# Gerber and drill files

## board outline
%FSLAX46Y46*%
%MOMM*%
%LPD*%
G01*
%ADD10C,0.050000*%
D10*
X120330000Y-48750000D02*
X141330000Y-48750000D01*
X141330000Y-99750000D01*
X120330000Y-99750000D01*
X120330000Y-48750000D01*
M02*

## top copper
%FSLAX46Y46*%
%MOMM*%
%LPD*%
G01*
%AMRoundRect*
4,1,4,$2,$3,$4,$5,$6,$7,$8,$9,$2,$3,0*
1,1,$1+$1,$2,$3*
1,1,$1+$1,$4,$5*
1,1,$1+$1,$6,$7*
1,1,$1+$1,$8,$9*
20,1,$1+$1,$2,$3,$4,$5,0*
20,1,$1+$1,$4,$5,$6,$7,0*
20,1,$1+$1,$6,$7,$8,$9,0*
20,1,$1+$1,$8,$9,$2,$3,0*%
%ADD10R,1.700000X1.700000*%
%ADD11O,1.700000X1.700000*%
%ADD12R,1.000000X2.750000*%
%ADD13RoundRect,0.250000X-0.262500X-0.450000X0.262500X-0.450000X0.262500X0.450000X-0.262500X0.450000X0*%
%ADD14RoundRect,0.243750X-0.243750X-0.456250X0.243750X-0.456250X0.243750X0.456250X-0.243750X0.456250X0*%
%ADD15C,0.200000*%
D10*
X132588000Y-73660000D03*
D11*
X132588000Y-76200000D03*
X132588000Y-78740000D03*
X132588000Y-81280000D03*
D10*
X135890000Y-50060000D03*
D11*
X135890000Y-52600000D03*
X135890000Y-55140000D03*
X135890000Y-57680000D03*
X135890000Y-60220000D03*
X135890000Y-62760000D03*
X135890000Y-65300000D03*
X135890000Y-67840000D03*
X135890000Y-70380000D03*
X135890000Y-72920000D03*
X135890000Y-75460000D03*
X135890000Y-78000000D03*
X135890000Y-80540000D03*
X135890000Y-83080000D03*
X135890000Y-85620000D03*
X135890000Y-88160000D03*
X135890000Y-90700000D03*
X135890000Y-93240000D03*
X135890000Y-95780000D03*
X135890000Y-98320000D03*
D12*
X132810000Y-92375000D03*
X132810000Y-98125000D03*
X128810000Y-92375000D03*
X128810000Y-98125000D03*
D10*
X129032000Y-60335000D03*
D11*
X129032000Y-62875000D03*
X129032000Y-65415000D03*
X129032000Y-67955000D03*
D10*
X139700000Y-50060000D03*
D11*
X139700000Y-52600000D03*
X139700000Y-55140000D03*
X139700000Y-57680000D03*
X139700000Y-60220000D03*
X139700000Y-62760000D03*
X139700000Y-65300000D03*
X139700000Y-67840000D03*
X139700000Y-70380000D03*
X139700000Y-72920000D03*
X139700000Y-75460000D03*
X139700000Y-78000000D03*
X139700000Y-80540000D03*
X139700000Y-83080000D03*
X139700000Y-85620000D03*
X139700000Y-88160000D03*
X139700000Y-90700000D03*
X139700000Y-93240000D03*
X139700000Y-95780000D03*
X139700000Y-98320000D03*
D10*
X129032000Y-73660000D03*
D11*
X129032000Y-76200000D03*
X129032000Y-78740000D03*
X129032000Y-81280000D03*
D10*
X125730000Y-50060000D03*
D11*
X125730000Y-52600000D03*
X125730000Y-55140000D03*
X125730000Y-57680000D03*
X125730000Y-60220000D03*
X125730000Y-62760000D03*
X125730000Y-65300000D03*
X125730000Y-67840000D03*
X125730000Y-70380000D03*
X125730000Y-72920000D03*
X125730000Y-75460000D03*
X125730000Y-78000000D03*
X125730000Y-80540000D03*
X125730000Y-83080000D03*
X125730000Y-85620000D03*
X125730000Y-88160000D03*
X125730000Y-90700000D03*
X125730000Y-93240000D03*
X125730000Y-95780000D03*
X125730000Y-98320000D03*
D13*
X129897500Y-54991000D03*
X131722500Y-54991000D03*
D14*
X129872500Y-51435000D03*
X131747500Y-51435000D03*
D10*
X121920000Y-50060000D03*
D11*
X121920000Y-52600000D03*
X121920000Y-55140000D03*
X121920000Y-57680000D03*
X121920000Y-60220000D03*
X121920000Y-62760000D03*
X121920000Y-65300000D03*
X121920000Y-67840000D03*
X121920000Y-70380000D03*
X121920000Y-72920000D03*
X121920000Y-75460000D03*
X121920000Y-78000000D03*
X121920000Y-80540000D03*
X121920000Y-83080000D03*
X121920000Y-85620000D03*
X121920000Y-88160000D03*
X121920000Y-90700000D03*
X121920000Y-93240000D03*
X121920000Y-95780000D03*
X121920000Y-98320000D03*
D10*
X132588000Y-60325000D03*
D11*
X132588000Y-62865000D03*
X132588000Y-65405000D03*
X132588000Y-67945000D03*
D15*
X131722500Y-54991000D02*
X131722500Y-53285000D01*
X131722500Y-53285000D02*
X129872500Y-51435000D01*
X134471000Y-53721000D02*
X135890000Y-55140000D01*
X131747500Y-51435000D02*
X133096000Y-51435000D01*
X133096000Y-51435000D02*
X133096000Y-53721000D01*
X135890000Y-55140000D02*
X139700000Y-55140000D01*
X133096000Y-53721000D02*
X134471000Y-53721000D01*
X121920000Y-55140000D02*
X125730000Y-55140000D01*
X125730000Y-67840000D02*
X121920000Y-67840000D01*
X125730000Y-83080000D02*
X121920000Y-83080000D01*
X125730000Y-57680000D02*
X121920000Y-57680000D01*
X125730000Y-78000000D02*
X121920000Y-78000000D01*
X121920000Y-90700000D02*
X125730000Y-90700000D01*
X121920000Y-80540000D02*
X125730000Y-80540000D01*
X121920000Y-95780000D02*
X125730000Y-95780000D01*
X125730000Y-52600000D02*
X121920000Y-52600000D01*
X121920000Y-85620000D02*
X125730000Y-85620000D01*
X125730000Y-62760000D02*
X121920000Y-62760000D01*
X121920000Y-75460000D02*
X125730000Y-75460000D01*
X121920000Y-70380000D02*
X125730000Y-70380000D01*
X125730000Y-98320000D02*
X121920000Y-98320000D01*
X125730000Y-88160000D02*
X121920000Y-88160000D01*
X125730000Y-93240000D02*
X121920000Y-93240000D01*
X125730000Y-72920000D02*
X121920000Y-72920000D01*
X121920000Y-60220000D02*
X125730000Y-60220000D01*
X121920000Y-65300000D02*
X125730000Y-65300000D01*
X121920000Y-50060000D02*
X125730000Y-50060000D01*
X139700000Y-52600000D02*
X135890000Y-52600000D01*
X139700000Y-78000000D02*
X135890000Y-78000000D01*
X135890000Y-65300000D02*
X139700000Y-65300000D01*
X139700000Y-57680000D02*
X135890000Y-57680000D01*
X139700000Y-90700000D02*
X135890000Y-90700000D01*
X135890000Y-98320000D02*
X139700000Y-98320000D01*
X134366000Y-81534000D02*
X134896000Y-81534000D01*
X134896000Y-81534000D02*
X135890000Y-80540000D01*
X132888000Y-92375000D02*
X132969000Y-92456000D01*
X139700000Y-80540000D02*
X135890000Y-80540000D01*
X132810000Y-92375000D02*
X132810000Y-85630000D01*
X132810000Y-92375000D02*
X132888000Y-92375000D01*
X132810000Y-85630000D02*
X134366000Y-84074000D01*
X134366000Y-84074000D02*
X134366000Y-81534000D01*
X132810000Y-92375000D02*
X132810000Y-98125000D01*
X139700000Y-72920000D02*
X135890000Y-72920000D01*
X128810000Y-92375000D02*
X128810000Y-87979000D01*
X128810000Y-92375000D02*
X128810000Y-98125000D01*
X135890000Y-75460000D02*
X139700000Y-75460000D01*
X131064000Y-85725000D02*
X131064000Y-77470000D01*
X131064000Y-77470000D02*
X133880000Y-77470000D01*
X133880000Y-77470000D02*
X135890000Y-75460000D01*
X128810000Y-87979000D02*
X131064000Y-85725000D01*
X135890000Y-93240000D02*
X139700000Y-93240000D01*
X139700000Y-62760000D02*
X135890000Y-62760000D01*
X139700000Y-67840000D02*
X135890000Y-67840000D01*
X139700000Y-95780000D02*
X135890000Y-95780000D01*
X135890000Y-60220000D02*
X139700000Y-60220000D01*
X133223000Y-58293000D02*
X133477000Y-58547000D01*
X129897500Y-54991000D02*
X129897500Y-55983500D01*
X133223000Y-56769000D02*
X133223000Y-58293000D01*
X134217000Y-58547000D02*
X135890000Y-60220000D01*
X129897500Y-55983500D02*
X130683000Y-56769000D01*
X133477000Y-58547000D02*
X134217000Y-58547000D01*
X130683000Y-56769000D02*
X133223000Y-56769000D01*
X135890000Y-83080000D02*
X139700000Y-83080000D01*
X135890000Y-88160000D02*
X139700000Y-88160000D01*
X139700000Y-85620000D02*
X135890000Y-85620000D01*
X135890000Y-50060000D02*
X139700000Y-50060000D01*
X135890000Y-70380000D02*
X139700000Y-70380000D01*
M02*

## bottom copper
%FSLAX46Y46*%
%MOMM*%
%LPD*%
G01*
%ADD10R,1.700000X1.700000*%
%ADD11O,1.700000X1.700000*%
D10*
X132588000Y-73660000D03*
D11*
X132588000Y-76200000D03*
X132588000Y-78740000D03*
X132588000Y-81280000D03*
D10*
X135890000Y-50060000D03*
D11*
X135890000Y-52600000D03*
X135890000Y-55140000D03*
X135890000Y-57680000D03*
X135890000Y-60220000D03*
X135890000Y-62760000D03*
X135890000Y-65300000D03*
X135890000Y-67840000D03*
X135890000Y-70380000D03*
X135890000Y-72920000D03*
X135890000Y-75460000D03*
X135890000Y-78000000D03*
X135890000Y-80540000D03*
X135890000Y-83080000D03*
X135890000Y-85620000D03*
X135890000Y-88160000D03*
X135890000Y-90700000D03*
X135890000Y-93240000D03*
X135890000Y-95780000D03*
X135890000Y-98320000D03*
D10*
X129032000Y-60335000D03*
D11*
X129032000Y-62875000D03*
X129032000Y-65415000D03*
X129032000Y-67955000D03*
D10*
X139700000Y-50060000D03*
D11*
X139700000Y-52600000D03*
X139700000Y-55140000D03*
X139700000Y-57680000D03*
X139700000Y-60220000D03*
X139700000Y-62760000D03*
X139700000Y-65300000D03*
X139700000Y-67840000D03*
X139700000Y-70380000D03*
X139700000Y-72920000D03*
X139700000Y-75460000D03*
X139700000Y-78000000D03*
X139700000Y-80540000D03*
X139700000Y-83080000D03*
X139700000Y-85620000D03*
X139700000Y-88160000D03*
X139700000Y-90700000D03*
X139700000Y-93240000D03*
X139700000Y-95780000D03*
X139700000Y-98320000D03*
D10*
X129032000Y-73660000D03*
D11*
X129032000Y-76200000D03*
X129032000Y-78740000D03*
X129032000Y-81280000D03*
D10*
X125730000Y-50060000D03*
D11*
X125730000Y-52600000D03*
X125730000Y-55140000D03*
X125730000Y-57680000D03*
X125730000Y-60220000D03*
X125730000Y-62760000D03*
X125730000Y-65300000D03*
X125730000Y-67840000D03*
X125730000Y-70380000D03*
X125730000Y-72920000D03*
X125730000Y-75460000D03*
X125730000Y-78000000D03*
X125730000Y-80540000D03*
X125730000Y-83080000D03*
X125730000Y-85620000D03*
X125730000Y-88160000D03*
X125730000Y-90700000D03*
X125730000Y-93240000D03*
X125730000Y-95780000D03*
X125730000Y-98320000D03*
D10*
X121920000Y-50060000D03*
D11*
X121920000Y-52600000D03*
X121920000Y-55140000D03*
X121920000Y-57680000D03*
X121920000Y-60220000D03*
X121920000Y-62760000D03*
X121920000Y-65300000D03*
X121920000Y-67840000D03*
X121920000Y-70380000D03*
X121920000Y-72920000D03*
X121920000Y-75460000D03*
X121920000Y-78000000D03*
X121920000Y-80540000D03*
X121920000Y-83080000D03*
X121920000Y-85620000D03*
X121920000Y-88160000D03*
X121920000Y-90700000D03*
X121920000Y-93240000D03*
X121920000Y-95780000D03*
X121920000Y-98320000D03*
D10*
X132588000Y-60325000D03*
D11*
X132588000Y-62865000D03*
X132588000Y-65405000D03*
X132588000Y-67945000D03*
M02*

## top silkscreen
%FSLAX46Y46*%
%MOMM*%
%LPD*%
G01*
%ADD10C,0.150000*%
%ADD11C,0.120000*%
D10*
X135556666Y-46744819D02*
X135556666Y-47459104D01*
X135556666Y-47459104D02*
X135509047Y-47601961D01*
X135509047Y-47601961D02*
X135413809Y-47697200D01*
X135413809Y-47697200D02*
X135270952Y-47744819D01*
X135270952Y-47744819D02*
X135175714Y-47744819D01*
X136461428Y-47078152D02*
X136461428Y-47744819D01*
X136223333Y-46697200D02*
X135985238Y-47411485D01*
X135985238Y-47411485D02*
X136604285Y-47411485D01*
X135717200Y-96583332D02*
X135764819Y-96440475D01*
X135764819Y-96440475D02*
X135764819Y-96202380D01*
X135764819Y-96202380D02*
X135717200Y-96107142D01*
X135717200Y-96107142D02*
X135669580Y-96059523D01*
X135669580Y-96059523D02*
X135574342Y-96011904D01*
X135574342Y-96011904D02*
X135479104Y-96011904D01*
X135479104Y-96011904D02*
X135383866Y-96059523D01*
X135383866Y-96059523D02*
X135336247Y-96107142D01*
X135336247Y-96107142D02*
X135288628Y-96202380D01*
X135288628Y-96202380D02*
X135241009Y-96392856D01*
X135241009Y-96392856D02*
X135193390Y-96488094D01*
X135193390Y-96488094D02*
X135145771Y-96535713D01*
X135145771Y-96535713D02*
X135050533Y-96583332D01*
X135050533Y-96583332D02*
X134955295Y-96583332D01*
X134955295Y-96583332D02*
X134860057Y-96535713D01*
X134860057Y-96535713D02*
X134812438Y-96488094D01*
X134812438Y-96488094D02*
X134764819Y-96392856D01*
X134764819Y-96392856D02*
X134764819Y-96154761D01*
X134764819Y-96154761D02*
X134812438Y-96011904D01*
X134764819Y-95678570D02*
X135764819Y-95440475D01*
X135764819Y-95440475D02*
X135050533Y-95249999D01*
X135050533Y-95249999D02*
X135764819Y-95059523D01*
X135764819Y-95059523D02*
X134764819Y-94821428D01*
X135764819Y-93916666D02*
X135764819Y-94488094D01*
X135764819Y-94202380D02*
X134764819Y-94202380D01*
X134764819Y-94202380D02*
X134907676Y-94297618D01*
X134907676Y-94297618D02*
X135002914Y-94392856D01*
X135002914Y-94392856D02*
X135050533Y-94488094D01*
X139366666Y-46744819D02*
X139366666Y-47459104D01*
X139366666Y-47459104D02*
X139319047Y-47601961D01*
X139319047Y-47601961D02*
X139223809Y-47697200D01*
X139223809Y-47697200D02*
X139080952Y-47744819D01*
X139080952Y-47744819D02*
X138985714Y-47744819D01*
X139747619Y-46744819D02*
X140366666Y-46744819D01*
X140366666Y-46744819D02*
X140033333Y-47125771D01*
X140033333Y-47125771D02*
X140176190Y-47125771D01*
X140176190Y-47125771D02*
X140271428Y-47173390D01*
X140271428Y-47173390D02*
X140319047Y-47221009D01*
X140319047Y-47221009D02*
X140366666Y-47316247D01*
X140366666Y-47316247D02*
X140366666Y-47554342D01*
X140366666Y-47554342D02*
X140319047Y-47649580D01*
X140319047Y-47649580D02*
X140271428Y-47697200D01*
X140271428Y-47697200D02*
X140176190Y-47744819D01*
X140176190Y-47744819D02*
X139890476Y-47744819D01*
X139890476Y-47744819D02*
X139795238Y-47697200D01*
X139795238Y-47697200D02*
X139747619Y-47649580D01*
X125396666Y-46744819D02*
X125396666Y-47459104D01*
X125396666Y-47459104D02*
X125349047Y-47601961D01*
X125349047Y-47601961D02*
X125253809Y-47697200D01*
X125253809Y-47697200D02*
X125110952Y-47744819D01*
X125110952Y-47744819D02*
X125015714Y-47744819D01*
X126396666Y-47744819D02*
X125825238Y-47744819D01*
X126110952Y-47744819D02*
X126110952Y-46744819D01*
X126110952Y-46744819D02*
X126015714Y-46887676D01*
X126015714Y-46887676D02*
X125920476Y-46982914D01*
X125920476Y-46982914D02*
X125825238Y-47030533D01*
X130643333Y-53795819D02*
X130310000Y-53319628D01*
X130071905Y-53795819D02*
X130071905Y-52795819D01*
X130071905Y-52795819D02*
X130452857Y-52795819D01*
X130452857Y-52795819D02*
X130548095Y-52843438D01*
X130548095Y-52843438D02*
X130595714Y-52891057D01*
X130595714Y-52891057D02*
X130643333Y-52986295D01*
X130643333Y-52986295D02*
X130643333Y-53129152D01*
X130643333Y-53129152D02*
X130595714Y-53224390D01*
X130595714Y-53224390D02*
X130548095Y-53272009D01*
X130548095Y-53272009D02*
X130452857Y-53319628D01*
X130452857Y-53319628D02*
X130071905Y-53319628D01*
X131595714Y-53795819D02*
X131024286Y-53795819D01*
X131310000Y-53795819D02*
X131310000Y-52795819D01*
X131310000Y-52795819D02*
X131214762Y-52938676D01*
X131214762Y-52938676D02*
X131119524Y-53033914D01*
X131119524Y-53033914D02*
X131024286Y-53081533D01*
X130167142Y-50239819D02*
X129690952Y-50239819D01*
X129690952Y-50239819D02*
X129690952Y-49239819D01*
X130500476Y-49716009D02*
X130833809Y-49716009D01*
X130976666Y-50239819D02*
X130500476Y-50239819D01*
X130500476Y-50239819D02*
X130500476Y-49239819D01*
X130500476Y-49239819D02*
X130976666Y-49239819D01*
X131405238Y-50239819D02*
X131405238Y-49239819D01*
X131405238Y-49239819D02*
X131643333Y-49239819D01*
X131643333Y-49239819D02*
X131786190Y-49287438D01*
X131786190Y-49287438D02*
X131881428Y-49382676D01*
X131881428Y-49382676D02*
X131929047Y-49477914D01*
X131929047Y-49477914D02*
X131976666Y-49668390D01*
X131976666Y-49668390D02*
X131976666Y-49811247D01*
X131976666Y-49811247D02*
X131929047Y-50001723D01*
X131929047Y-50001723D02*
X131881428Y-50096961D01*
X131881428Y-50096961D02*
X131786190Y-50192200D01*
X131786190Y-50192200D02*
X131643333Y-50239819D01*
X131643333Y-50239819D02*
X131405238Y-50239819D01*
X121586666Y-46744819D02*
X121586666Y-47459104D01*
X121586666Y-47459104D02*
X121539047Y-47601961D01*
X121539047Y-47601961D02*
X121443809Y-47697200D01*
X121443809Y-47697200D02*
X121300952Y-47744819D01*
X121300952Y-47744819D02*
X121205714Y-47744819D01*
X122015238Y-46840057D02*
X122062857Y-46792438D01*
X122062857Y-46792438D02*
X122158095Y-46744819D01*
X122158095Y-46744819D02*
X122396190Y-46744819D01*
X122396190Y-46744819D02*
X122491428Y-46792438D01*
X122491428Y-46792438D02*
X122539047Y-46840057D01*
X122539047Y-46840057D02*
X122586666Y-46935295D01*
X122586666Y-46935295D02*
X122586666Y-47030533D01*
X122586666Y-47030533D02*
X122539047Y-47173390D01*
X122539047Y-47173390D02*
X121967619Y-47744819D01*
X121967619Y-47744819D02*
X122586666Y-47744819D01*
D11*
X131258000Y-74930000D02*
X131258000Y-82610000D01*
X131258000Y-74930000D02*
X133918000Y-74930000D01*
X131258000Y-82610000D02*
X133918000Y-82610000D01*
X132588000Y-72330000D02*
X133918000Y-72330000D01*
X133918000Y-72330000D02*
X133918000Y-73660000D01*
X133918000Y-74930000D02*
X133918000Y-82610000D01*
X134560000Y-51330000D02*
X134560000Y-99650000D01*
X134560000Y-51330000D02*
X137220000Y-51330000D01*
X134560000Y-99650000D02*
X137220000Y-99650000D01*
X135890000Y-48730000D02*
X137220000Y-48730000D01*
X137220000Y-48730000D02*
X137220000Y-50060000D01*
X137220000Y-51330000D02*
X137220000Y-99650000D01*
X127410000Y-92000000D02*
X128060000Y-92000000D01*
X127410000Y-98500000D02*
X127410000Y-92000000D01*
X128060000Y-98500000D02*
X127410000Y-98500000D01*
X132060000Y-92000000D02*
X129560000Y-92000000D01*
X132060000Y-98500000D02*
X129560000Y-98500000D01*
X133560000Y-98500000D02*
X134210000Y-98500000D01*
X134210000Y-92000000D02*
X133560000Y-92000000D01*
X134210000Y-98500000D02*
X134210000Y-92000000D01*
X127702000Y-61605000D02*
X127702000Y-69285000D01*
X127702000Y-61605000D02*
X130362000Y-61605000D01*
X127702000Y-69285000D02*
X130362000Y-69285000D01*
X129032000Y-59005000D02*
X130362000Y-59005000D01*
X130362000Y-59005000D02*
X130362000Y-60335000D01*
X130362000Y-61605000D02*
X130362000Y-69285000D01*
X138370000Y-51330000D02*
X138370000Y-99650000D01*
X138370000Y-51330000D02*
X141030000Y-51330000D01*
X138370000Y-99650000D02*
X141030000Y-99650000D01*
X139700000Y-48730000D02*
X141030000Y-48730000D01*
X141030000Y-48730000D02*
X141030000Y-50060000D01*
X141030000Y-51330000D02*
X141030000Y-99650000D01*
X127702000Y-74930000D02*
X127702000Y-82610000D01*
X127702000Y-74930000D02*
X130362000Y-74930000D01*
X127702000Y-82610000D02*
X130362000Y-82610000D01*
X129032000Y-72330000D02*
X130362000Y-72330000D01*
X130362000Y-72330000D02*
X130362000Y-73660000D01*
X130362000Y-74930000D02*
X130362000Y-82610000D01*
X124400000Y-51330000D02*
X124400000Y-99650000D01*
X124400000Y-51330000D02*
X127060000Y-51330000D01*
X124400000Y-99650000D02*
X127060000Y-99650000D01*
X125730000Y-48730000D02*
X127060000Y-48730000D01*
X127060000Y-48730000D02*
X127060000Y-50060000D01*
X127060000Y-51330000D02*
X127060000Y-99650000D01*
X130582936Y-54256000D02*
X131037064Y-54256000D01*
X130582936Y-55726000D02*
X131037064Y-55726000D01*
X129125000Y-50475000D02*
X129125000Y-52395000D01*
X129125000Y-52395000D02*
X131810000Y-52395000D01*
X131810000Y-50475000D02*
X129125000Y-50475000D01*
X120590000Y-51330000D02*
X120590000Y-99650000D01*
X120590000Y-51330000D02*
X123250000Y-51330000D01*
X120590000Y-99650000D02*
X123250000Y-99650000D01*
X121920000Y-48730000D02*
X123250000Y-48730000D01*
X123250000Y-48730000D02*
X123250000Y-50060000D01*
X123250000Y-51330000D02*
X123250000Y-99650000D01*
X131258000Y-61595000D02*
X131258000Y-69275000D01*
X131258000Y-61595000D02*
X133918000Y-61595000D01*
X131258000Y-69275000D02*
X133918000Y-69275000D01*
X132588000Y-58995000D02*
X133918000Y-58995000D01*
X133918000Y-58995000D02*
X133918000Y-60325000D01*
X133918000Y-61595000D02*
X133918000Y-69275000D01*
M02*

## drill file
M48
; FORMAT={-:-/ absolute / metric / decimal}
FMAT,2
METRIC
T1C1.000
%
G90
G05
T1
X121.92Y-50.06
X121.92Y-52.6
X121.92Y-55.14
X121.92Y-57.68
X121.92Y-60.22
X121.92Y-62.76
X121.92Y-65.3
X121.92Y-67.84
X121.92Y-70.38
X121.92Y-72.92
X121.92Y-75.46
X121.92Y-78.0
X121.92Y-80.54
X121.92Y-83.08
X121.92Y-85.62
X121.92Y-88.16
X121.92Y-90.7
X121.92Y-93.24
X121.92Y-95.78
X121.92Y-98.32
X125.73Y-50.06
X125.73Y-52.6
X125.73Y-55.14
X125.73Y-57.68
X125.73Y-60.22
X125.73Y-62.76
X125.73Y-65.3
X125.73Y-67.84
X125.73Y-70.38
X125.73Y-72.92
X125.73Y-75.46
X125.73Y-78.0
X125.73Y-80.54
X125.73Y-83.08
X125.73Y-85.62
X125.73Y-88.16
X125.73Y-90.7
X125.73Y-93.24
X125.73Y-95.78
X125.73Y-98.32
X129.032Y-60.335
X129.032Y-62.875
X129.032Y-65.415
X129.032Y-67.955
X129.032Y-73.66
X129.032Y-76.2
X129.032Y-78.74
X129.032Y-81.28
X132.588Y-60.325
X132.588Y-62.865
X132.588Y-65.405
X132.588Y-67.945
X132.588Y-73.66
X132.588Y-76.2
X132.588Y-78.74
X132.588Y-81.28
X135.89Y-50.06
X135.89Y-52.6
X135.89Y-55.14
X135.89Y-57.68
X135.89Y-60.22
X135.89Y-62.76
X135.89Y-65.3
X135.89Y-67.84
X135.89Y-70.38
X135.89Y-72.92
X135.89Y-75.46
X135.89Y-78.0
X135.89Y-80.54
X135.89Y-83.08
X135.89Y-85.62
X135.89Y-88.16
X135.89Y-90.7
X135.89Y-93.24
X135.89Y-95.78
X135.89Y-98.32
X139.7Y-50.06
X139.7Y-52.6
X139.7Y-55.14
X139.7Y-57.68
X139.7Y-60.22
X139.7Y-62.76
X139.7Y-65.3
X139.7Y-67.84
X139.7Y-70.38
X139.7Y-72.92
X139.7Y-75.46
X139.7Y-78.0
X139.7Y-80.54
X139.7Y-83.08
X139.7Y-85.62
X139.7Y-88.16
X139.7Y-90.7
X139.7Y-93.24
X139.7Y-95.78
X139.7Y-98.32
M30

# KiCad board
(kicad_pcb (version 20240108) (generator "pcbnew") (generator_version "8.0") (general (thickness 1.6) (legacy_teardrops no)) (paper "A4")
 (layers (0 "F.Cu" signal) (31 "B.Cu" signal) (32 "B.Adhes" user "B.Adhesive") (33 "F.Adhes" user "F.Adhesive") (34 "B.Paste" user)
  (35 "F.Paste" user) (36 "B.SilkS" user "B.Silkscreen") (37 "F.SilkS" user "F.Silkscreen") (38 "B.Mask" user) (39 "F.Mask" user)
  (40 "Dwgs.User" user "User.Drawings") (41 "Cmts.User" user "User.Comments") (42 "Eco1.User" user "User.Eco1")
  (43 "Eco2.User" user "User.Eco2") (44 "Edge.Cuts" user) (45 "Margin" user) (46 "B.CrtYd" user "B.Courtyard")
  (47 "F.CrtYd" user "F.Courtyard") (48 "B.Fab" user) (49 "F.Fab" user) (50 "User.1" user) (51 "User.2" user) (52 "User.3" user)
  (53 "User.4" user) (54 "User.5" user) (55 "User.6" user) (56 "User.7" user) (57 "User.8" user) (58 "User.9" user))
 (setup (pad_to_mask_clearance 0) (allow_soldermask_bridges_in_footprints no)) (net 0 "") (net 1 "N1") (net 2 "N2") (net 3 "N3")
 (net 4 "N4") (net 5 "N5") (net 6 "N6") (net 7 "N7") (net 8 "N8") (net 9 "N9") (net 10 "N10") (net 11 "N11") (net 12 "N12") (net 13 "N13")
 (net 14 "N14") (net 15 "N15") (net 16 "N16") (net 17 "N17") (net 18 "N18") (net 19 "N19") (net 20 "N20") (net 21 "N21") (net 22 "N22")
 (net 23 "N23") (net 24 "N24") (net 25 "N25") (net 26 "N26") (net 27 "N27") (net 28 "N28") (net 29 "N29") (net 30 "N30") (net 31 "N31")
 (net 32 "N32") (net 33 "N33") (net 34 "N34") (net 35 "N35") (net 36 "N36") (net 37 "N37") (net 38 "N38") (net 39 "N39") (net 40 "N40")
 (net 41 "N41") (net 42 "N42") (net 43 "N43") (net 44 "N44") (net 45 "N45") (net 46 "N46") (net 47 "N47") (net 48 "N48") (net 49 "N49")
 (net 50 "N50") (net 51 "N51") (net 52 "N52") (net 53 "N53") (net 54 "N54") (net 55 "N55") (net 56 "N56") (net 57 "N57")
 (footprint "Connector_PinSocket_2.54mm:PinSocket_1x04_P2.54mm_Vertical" (layer "F.Cu") (at 132.588 73.66)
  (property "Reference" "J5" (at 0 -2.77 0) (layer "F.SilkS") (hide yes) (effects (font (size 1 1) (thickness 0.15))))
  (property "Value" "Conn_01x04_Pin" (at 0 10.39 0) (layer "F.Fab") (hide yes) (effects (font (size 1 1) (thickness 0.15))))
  (fp_line (start -1.33 1.27) (end -1.33 8.95) (stroke (width 0.12) (type solid)) (layer "F.SilkS"))
  (fp_line (start -1.33 1.27) (end 1.33 1.27) (stroke (width 0.12) (type solid)) (layer "F.SilkS"))
  (fp_line (start -1.33 8.95) (end 1.33 8.95) (stroke (width 0.12) (type solid)) (layer "F.SilkS"))
  (fp_line (start 0 -1.33) (end 1.33 -1.33) (stroke (width 0.12) (type solid)) (layer "F.SilkS"))
  (fp_line (start 1.33 -1.33) (end 1.33 0) (stroke (width 0.12) (type solid)) (layer "F.SilkS"))
  (fp_line (start 1.33 1.27) (end 1.33 8.95) (stroke (width 0.12) (type solid)) (layer "F.SilkS"))
  (pad "1" thru_hole rect (at 0 0) (size 1.7 1.7) (drill 1) (layers "*.Cu" "*.Mask") (remove_unused_layers no) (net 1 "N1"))
  (pad "2" thru_hole oval (at 0 2.54) (size 1.7 1.7) (drill 1) (layers "*.Cu" "*.Mask") (remove_unused_layers no) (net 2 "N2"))
  (pad "3" thru_hole oval (at 0 5.08) (size 1.7 1.7) (drill 1) (layers "*.Cu" "*.Mask") (remove_unused_layers no) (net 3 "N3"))
  (pad "4" thru_hole oval (at 0 7.62) (size 1.7 1.7) (drill 1) (layers "*.Cu" "*.Mask") (remove_unused_layers no) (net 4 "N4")))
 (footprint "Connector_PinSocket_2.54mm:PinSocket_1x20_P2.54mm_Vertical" (layer "F.Cu") (at 135.89 50.06)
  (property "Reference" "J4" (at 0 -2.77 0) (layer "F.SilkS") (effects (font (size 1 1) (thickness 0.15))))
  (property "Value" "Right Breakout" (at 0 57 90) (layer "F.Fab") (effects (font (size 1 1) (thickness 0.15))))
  (fp_line (start -1.33 1.27) (end -1.33 49.59) (stroke (width 0.12) (type solid)) (layer "F.SilkS"))
  (fp_line (start -1.33 1.27) (end 1.33 1.27) (stroke (width 0.12) (type solid)) (layer "F.SilkS"))
  (fp_line (start -1.33 49.59) (end 1.33 49.59) (stroke (width 0.12) (type solid)) (layer "F.SilkS"))
  (fp_line (start 0 -1.33) (end 1.33 -1.33) (stroke (width 0.12) (type solid)) (layer "F.SilkS"))
  (fp_line (start 1.33 -1.33) (end 1.33 0) (stroke (width 0.12) (type solid)) (layer "F.SilkS"))
  (fp_line (start 1.33 1.27) (end 1.33 49.59) (stroke (width 0.12) (type solid)) (layer "F.SilkS"))
  (pad "1" thru_hole rect (at 0 0) (size 1.7 1.7) (drill 1) (layers "*.Cu" "*.Mask") (remove_unused_layers no) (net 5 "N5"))
  (pad "2" thru_hole oval (at 0 2.54) (size 1.7 1.7) (drill 1) (layers "*.Cu" "*.Mask") (remove_unused_layers no) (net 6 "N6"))
  (pad "3" thru_hole oval (at 0 5.08) (size 1.7 1.7) (drill 1) (layers "*.Cu" "*.Mask") (remove_unused_layers no) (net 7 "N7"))
  (pad "4" thru_hole oval (at 0 7.62) (size 1.7 1.7) (drill 1) (layers "*.Cu" "*.Mask") (remove_unused_layers no) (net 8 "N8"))
  (pad "5" thru_hole oval (at 0 10.16) (size 1.7 1.7) (drill 1) (layers "*.Cu" "*.Mask") (remove_unused_layers no) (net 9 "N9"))
  (pad "6" thru_hole oval (at 0 12.7) (size 1.7 1.7) (drill 1) (layers "*.Cu" "*.Mask") (remove_unused_layers no) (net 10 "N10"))
  (pad "7" thru_hole oval (at 0 15.24) (size 1.7 1.7) (drill 1) (layers "*.Cu" "*.Mask") (remove_unused_layers no) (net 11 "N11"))
  (pad "8" thru_hole oval (at 0 17.78) (size 1.7 1.7) (drill 1) (layers "*.Cu" "*.Mask") (remove_unused_layers no) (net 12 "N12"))
  (pad "9" thru_hole oval (at 0 20.32) (size 1.7 1.7) (drill 1) (layers "*.Cu" "*.Mask") (remove_unused_layers no) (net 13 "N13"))
  (pad "10" thru_hole oval (at 0 22.86) (size 1.7 1.7) (drill 1) (layers "*.Cu" "*.Mask") (remove_unused_layers no) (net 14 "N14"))
  (pad "11" thru_hole oval (at 0 25.4) (size 1.7 1.7) (drill 1) (layers "*.Cu" "*.Mask") (remove_unused_layers no) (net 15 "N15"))
  (pad "12" thru_hole oval (at 0 27.94) (size 1.7 1.7) (drill 1) (layers "*.Cu" "*.Mask") (remove_unused_layers no) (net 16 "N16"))
  (pad "13" thru_hole oval (at 0 30.48) (size 1.7 1.7) (drill 1) (layers "*.Cu" "*.Mask") (remove_unused_layers no) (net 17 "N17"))
  (pad "14" thru_hole oval (at 0 33.02) (size 1.7 1.7) (drill 1) (layers "*.Cu" "*.Mask") (remove_unused_layers no) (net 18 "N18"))
  (pad "15" thru_hole oval (at 0 35.56) (size 1.7 1.7) (drill 1) (layers "*.Cu" "*.Mask") (remove_unused_layers no) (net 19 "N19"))
  (pad "16" thru_hole oval (at 0 38.1) (size 1.7 1.7) (drill 1) (layers "*.Cu" "*.Mask") (remove_unused_layers no) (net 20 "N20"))
  (pad "17" thru_hole oval (at 0 40.64) (size 1.7 1.7) (drill 1) (layers "*.Cu" "*.Mask") (remove_unused_layers no) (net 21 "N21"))
  (pad "18" thru_hole oval (at 0 43.18) (size 1.7 1.7) (drill 1) (layers "*.Cu" "*.Mask") (remove_unused_layers no) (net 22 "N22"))
  (pad "19" thru_hole oval (at 0 45.72) (size 1.7 1.7) (drill 1) (layers "*.Cu" "*.Mask") (remove_unused_layers no) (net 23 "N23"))
  (pad "20" thru_hole oval (at 0 48.26) (size 1.7 1.7) (drill 1) (layers "*.Cu" "*.Mask") (remove_unused_layers no) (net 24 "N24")))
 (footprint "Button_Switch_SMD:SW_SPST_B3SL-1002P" (layer "F.Cu") (at 130.81 95.25 -90)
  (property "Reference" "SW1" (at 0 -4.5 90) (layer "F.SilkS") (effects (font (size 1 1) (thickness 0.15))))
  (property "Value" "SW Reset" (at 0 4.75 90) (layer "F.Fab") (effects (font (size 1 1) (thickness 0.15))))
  (fp_line (start -3.25 3.4) (end -3.25 2.75) (stroke (width 0.12) (type solid)) (layer "F.SilkS"))
  (fp_line (start 3.25 3.4) (end -3.25 3.4) (stroke (width 0.12) (type solid)) (layer "F.SilkS"))
  (fp_line (start 3.25 2.75) (end 3.25 3.4) (stroke (width 0.12) (type solid)) (layer "F.SilkS"))
  (fp_line (start -3.25 -1.25) (end -3.25 1.25) (stroke (width 0.12) (type solid)) (layer "F.SilkS"))
  (fp_line (start 3.25 -1.25) (end 3.25 1.25) (stroke (width 0.12) (type solid)) (layer "F.SilkS"))
  (fp_line (start 3.25 -2.75) (end 3.25 -3.4) (stroke (width 0.12) (type solid)) (layer "F.SilkS"))
  (fp_line (start -3.25 -3.4) (end -3.25 -2.75) (stroke (width 0.12) (type solid)) (layer "F.SilkS"))
  (fp_line (start 3.25 -3.4) (end -3.25 -3.4) (stroke (width 0.12) (type solid)) (layer "F.SilkS"))
  (pad "1" smd rect (at -2.875 -2 270) (size 2.75 1) (layers "F.Cu" "F.Paste" "F.Mask") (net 17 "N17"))
  (pad "1" smd rect (at 2.875 -2 270) (size 2.75 1) (layers "F.Cu" "F.Paste" "F.Mask") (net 17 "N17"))
  (pad "2" smd rect (at -2.875 2 270) (size 2.75 1) (layers "F.Cu" "F.Paste" "F.Mask") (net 15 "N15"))
  (pad "2" smd rect (at 2.875 2 270) (size 2.75 1) (layers "F.Cu" "F.Paste" "F.Mask") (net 15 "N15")))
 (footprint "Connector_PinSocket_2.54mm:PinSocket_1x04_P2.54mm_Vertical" (layer "F.Cu") (at 129.032 60.335)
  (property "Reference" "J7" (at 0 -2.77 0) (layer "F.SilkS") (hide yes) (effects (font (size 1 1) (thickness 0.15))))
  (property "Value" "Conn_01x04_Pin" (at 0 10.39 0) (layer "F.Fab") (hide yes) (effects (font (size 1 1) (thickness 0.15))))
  (fp_line (start -1.33 1.27) (end -1.33 8.95) (stroke (width 0.12) (type solid)) (layer "F.SilkS"))
  (fp_line (start -1.33 1.27) (end 1.33 1.27) (stroke (width 0.12) (type solid)) (layer "F.SilkS"))
  (fp_line (start -1.33 8.95) (end 1.33 8.95) (stroke (width 0.12) (type solid)) (layer "F.SilkS"))
  (fp_line (start 0 -1.33) (end 1.33 -1.33) (stroke (width 0.12) (type solid)) (layer "F.SilkS"))
  (fp_line (start 1.33 -1.33) (end 1.33 0) (stroke (width 0.12) (type solid)) (layer "F.SilkS"))
  (fp_line (start 1.33 1.27) (end 1.33 8.95) (stroke (width 0.12) (type solid)) (layer "F.SilkS"))
  (pad "1" thru_hole rect (at 0 0) (size 1.7 1.7) (drill 1) (layers "*.Cu" "*.Mask") (remove_unused_layers no) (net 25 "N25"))
  (pad "2" thru_hole oval (at 0 2.54) (size 1.7 1.7) (drill 1) (layers "*.Cu" "*.Mask") (remove_unused_layers no) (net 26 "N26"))
  (pad "3" thru_hole oval (at 0 5.08) (size 1.7 1.7) (drill 1) (layers "*.Cu" "*.Mask") (remove_unused_layers no) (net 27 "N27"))
  (pad "4" thru_hole oval (at 0 7.62) (size 1.7 1.7) (drill 1) (layers "*.Cu" "*.Mask") (remove_unused_layers no) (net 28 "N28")))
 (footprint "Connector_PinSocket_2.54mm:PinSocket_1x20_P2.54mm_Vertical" (layer "F.Cu") (at 139.7 50.06)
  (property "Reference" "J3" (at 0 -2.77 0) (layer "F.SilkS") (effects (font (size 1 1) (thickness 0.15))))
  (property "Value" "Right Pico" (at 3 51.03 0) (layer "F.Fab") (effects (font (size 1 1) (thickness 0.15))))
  (fp_line (start -1.33 1.27) (end -1.33 49.59) (stroke (width 0.12) (type solid)) (layer "F.SilkS"))
  (fp_line (start -1.33 1.27) (end 1.33 1.27) (stroke (width 0.12) (type solid)) (layer "F.SilkS"))
  (fp_line (start -1.33 49.59) (end 1.33 49.59) (stroke (width 0.12) (type solid)) (layer "F.SilkS"))
  (fp_line (start 0 -1.33) (end 1.33 -1.33) (stroke (width 0.12) (type solid)) (layer "F.SilkS"))
  (fp_line (start 1.33 -1.33) (end 1.33 0) (stroke (width 0.12) (type solid)) (layer "F.SilkS"))
  (fp_line (start 1.33 1.27) (end 1.33 49.59) (stroke (width 0.12) (type solid)) (layer "F.SilkS"))
  (pad "1" thru_hole rect (at 0 0) (size 1.7 1.7) (drill 1) (layers "*.Cu" "*.Mask") (remove_unused_layers no) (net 5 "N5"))
  (pad "2" thru_hole oval (at 0 2.54) (size 1.7 1.7) (drill 1) (layers "*.Cu" "*.Mask") (remove_unused_layers no) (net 6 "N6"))
  (pad "3" thru_hole oval (at 0 5.08) (size 1.7 1.7) (drill 1) (layers "*.Cu" "*.Mask") (remove_unused_layers no) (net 7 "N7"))
  (pad "4" thru_hole oval (at 0 7.62) (size 1.7 1.7) (drill 1) (layers "*.Cu" "*.Mask") (remove_unused_layers no) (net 8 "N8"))
  (pad "5" thru_hole oval (at 0 10.16) (size 1.7 1.7) (drill 1) (layers "*.Cu" "*.Mask") (remove_unused_layers no) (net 9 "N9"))
  (pad "6" thru_hole oval (at 0 12.7) (size 1.7 1.7) (drill 1) (layers "*.Cu" "*.Mask") (remove_unused_layers no) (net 10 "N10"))
  (pad "7" thru_hole oval (at 0 15.24) (size 1.7 1.7) (drill 1) (layers "*.Cu" "*.Mask") (remove_unused_layers no) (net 11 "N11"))
  (pad "8" thru_hole oval (at 0 17.78) (size 1.7 1.7) (drill 1) (layers "*.Cu" "*.Mask") (remove_unused_layers no) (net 12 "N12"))
  (pad "9" thru_hole oval (at 0 20.32) (size 1.7 1.7) (drill 1) (layers "*.Cu" "*.Mask") (remove_unused_layers no) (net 13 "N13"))
  (pad "10" thru_hole oval (at 0 22.86) (size 1.7 1.7) (drill 1) (layers "*.Cu" "*.Mask") (remove_unused_layers no) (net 14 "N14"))
  (pad "11" thru_hole oval (at 0 25.4) (size 1.7 1.7) (drill 1) (layers "*.Cu" "*.Mask") (remove_unused_layers no) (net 15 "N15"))
  (pad "12" thru_hole oval (at 0 27.94) (size 1.7 1.7) (drill 1) (layers "*.Cu" "*.Mask") (remove_unused_layers no) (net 16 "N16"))
  (pad "13" thru_hole oval (at 0 30.48) (size 1.7 1.7) (drill 1) (layers "*.Cu" "*.Mask") (remove_unused_layers no) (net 17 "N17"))
  (pad "14" thru_hole oval (at 0 33.02) (size 1.7 1.7) (drill 1) (layers "*.Cu" "*.Mask") (remove_unused_layers no) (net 18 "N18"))
  (pad "15" thru_hole oval (at 0 35.56) (size 1.7 1.7) (drill 1) (layers "*.Cu" "*.Mask") (remove_unused_layers no) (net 19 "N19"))
  (pad "16" thru_hole oval (at 0 38.1) (size 1.7 1.7) (drill 1) (layers "*.Cu" "*.Mask") (remove_unused_layers no) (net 20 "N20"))
  (pad "17" thru_hole oval (at 0 40.64) (size 1.7 1.7) (drill 1) (layers "*.Cu" "*.Mask") (remove_unused_layers no) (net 21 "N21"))
  (pad "18" thru_hole oval (at 0 43.18) (size 1.7 1.7) (drill 1) (layers "*.Cu" "*.Mask") (remove_unused_layers no) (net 22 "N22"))
  (pad "19" thru_hole oval (at 0 45.72) (size 1.7 1.7) (drill 1) (layers "*.Cu" "*.Mask") (remove_unused_layers no) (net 23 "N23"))
  (pad "20" thru_hole oval (at 0 48.26) (size 1.7 1.7) (drill 1) (layers "*.Cu" "*.Mask") (remove_unused_layers no) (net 24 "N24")))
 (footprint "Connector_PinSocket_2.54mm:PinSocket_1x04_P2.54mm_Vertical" (layer "F.Cu") (at 129.032 73.66)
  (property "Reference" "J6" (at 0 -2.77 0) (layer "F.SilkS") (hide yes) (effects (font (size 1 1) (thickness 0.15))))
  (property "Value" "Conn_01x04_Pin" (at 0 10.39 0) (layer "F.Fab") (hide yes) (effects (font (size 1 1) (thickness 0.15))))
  (fp_line (start -1.33 1.27) (end -1.33 8.95) (stroke (width 0.12) (type solid)) (layer "F.SilkS"))
  (fp_line (start -1.33 1.27) (end 1.33 1.27) (stroke (width 0.12) (type solid)) (layer "F.SilkS"))
  (fp_line (start -1.33 8.95) (end 1.33 8.95) (stroke (width 0.12) (type solid)) (layer "F.SilkS"))
  (fp_line (start 0 -1.33) (end 1.33 -1.33) (stroke (width 0.12) (type solid)) (layer "F.SilkS"))
  (fp_line (start 1.33 -1.33) (end 1.33 0) (stroke (width 0.12) (type solid)) (layer "F.SilkS"))
  (fp_line (start 1.33 1.27) (end 1.33 8.95) (stroke (width 0.12) (type solid)) (layer "F.SilkS"))
  (pad "1" thru_hole rect (at 0 0) (size 1.7 1.7) (drill 1) (layers "*.Cu" "*.Mask") (remove_unused_layers no) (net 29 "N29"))
  (pad "2" thru_hole oval (at 0 2.54) (size 1.7 1.7) (drill 1) (layers "*.Cu" "*.Mask") (remove_unused_layers no) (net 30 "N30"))
  (pad "3" thru_hole oval (at 0 5.08) (size 1.7 1.7) (drill 1) (layers "*.Cu" "*.Mask") (remove_unused_layers no) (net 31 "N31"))
  (pad "4" thru_hole oval (at 0 7.62) (size 1.7 1.7) (drill 1) (layers "*.Cu" "*.Mask") (remove_unused_layers no) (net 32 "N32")))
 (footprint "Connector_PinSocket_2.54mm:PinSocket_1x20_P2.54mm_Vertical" (layer "F.Cu") (at 125.73 50.06)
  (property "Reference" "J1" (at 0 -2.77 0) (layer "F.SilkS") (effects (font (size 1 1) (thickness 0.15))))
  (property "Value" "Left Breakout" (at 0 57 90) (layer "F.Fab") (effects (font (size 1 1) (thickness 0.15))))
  (fp_line (start -1.33 1.27) (end -1.33 49.59) (stroke (width 0.12) (type solid)) (layer "F.SilkS"))
  (fp_line (start -1.33 1.27) (end 1.33 1.27) (stroke (width 0.12) (type solid)) (layer "F.SilkS"))
  (fp_line (start -1.33 49.59) (end 1.33 49.59) (stroke (width 0.12) (type solid)) (layer "F.SilkS"))
  (fp_line (start 0 -1.33) (end 1.33 -1.33) (stroke (width 0.12) (type solid)) (layer "F.SilkS"))
  (fp_line (start 1.33 -1.33) (end 1.33 0) (stroke (width 0.12) (type solid)) (layer "F.SilkS"))
  (fp_line (start 1.33 1.27) (end 1.33 49.59) (stroke (width 0.12) (type solid)) (layer "F.SilkS"))
  (pad "1" thru_hole rect (at 0 0) (size 1.7 1.7) (drill 1) (layers "*.Cu" "*.Mask") (remove_unused_layers no) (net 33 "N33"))
  (pad "2" thru_hole oval (at 0 2.54) (size 1.7 1.7) (drill 1) (layers "*.Cu" "*.Mask") (remove_unused_layers no) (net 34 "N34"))
  (pad "3" thru_hole oval (at 0 5.08) (size 1.7 1.7) (drill 1) (layers "*.Cu" "*.Mask") (remove_unused_layers no) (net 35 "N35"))
  (pad "4" thru_hole oval (at 0 7.62) (size 1.7 1.7) (drill 1) (layers "*.Cu" "*.Mask") (remove_unused_layers no) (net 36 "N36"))
  (pad "5" thru_hole oval (at 0 10.16) (size 1.7 1.7) (drill 1) (layers "*.Cu" "*.Mask") (remove_unused_layers no) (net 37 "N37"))
  (pad "6" thru_hole oval (at 0 12.7) (size 1.7 1.7) (drill 1) (layers "*.Cu" "*.Mask") (remove_unused_layers no) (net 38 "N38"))
  (pad "7" thru_hole oval (at 0 15.24) (size 1.7 1.7) (drill 1) (layers "*.Cu" "*.Mask") (remove_unused_layers no) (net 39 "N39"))
  (pad "8" thru_hole oval (at 0 17.78) (size 1.7 1.7) (drill 1) (layers "*.Cu" "*.Mask") (remove_unused_layers no) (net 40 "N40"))
  (pad "9" thru_hole oval (at 0 20.32) (size 1.7 1.7) (drill 1) (layers "*.Cu" "*.Mask") (remove_unused_layers no) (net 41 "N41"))
  (pad "10" thru_hole oval (at 0 22.86) (size 1.7 1.7) (drill 1) (layers "*.Cu" "*.Mask") (remove_unused_layers no) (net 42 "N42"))
  (pad "11" thru_hole oval (at 0 25.4) (size 1.7 1.7) (drill 1) (layers "*.Cu" "*.Mask") (remove_unused_layers no) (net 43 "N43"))
  (pad "12" thru_hole oval (at 0 27.94) (size 1.7 1.7) (drill 1) (layers "*.Cu" "*.Mask") (remove_unused_layers no) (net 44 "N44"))
  (pad "13" thru_hole oval (at 0 30.48) (size 1.7 1.7) (drill 1) (layers "*.Cu" "*.Mask") (remove_unused_layers no) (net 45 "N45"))
  (pad "14" thru_hole oval (at 0 33.02) (size 1.7 1.7) (drill 1) (layers "*.Cu" "*.Mask") (remove_unused_layers no) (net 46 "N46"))
  (pad "15" thru_hole oval (at 0 35.56) (size 1.7 1.7) (drill 1) (layers "*.Cu" "*.Mask") (remove_unused_layers no) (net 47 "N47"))
  (pad "16" thru_hole oval (at 0 38.1) (size 1.7 1.7) (drill 1) (layers "*.Cu" "*.Mask") (remove_unused_layers no) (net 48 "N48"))
  (pad "17" thru_hole oval (at 0 40.64) (size 1.7 1.7) (drill 1) (layers "*.Cu" "*.Mask") (remove_unused_layers no) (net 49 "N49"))
  (pad "18" thru_hole oval (at 0 43.18) (size 1.7 1.7) (drill 1) (layers "*.Cu" "*.Mask") (remove_unused_layers no) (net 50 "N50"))
  (pad "19" thru_hole oval (at 0 45.72) (size 1.7 1.7) (drill 1) (layers "*.Cu" "*.Mask") (remove_unused_layers no) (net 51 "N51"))
  (pad "20" thru_hole oval (at 0 48.26) (size 1.7 1.7) (drill 1) (layers "*.Cu" "*.Mask") (remove_unused_layers no) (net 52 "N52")))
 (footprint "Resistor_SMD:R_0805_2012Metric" (layer "F.Cu") (at 130.81 54.991)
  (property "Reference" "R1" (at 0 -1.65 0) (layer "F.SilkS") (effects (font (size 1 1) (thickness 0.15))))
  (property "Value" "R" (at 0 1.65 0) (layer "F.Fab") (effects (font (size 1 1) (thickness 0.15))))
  (fp_line (start -0.227064 -0.735) (end 0.227064 -0.735) (stroke (width 0.12) (type solid)) (layer "F.SilkS"))
  (fp_line (start -0.227064 0.735) (end 0.227064 0.735) (stroke (width 0.12) (type solid)) (layer "F.SilkS"))
  (pad "1" smd roundrect (at -0.9125 0) (size 1.025 1.4) (layers "F.Cu" "F.Paste" "F.Mask") (roundrect_rratio 0.243902) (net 9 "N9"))
  (pad "2" smd roundrect (at 0.9125 0) (size 1.025 1.4) (layers "F.Cu" "F.Paste" "F.Mask") (roundrect_rratio 0.243902) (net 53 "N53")))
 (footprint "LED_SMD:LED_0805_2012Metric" (layer "F.Cu") (at 130.81 51.435)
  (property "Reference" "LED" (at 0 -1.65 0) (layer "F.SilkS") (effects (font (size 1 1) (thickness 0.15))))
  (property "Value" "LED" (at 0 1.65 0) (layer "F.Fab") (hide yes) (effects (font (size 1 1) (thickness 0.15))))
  (fp_line (start -1.685 -0.96) (end -1.685 0.96) (stroke (width 0.12) (type solid)) (layer "F.SilkS"))
  (fp_line (start -1.685 0.96) (end 1 0.96) (stroke (width 0.12) (type solid)) (layer "F.SilkS"))
  (fp_line (start 1 -0.96) (end -1.685 -0.96) (stroke (width 0.12) (type solid)) (layer "F.SilkS"))
  (pad "1" smd roundrect (at -0.9375 0) (size 0.975 1.4) (layers "F.Cu" "F.Paste" "F.Mask") (roundrect_rratio 0.25) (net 53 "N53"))
  (pad "2" smd roundrect (at 0.9375 0) (size 0.975 1.4) (layers "F.Cu" "F.Paste" "F.Mask") (roundrect_rratio 0.25) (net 7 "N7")))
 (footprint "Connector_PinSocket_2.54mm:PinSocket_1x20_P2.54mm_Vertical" (layer "F.Cu") (at 121.92 50.06)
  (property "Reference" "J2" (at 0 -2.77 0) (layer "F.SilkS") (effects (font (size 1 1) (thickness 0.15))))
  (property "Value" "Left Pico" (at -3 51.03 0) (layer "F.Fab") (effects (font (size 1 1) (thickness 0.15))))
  (fp_line (start -1.33 1.27) (end -1.33 49.59) (stroke (width 0.12) (type solid)) (layer "F.SilkS"))
  (fp_line (start -1.33 1.27) (end 1.33 1.27) (stroke (width 0.12) (type solid)) (layer "F.SilkS"))
  (fp_line (start -1.33 49.59) (end 1.33 49.59) (stroke (width 0.12) (type solid)) (layer "F.SilkS"))
  (fp_line (start 0 -1.33) (end 1.33 -1.33) (stroke (width 0.12) (type solid)) (layer "F.SilkS"))
  (fp_line (start 1.33 -1.33) (end 1.33 0) (stroke (width 0.12) (type solid)) (layer "F.SilkS"))
  (fp_line (start 1.33 1.27) (end 1.33 49.59) (stroke (width 0.12) (type solid)) (layer "F.SilkS"))
  (pad "1" thru_hole rect (at 0 0) (size 1.7 1.7) (drill 1) (layers "*.Cu" "*.Mask") (remove_unused_layers no) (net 33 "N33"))
  (pad "2" thru_hole oval (at 0 2.54) (size 1.7 1.7) (drill 1) (layers "*.Cu" "*.Mask") (remove_unused_layers no) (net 34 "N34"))
  (pad "3" thru_hole oval (at 0 5.08) (size 1.7 1.7) (drill 1) (layers "*.Cu" "*.Mask") (remove_unused_layers no) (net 35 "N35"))
  (pad "4" thru_hole oval (at 0 7.62) (size 1.7 1.7) (drill 1) (layers "*.Cu" "*.Mask") (remove_unused_layers no) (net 36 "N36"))
  (pad "5" thru_hole oval (at 0 10.16) (size 1.7 1.7) (drill 1) (layers "*.Cu" "*.Mask") (remove_unused_layers no) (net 37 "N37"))
  (pad "6" thru_hole oval (at 0 12.7) (size 1.7 1.7) (drill 1) (layers "*.Cu" "*.Mask") (remove_unused_layers no) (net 38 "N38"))
  (pad "7" thru_hole oval (at 0 15.24) (size 1.7 1.7) (drill 1) (layers "*.Cu" "*.Mask") (remove_unused_layers no) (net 39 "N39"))
  (pad "8" thru_hole oval (at 0 17.78) (size 1.7 1.7) (drill 1) (layers "*.Cu" "*.Mask") (remove_unused_layers no) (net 40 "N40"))
  (pad "9" thru_hole oval (at 0 20.32) (size 1.7 1.7) (drill 1) (layers "*.Cu" "*.Mask") (remove_unused_layers no) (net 41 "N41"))
  (pad "10" thru_hole oval (at 0 22.86) (size 1.7 1.7) (drill 1) (layers "*.Cu" "*.Mask") (remove_unused_layers no) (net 42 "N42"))
  (pad "11" thru_hole oval (at 0 25.4) (size 1.7 1.7) (drill 1) (layers "*.Cu" "*.Mask") (remove_unused_layers no) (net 43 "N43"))
  (pad "12" thru_hole oval (at 0 27.94) (size 1.7 1.7) (drill 1) (layers "*.Cu" "*.Mask") (remove_unused_layers no) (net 44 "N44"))
  (pad "13" thru_hole oval (at 0 30.48) (size 1.7 1.7) (drill 1) (layers "*.Cu" "*.Mask") (remove_unused_layers no) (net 45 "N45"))
  (pad "14" thru_hole oval (at 0 33.02) (size 1.7 1.7) (drill 1) (layers "*.Cu" "*.Mask") (remove_unused_layers no) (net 46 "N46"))
  (pad "15" thru_hole oval (at 0 35.56) (size 1.7 1.7) (drill 1) (layers "*.Cu" "*.Mask") (remove_unused_layers no) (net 47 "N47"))
  (pad "16" thru_hole oval (at 0 38.1) (size 1.7 1.7) (drill 1) (layers "*.Cu" "*.Mask") (remove_unused_layers no) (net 48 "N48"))
  (pad "17" thru_hole oval (at 0 40.64) (size 1.7 1.7) (drill 1) (layers "*.Cu" "*.Mask") (remove_unused_layers no) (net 49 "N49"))
  (pad "18" thru_hole oval (at 0 43.18) (size 1.7 1.7) (drill 1) (layers "*.Cu" "*.Mask") (remove_unused_layers no) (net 50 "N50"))
  (pad "19" thru_hole oval (at 0 45.72) (size 1.7 1.7) (drill 1) (layers "*.Cu" "*.Mask") (remove_unused_layers no) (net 51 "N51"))
  (pad "20" thru_hole oval (at 0 48.26) (size 1.7 1.7) (drill 1) (layers "*.Cu" "*.Mask") (remove_unused_layers no) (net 52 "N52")))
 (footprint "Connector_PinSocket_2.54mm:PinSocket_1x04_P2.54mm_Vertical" (layer "F.Cu") (at 132.588 60.325)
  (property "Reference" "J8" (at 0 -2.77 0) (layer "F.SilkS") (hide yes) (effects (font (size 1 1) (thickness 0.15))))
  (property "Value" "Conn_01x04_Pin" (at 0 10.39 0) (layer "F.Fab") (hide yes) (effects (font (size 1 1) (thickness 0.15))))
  (fp_line (start -1.33 1.27) (end -1.33 8.95) (stroke (width 0.12) (type solid)) (layer "F.SilkS"))
  (fp_line (start -1.33 1.27) (end 1.33 1.27) (stroke (width 0.12) (type solid)) (layer "F.SilkS"))
  (fp_line (start -1.33 8.95) (end 1.33 8.95) (stroke (width 0.12) (type solid)) (layer "F.SilkS"))
  (fp_line (start 0 -1.33) (end 1.33 -1.33) (stroke (width 0.12) (type solid)) (layer "F.SilkS"))
  (fp_line (start 1.33 -1.33) (end 1.33 0) (stroke (width 0.12) (type solid)) (layer "F.SilkS"))
  (fp_line (start 1.33 1.27) (end 1.33 8.95) (stroke (width 0.12) (type solid)) (layer "F.SilkS"))
  (pad "1" thru_hole rect (at 0 0) (size 1.7 1.7) (drill 1) (layers "*.Cu" "*.Mask") (remove_unused_layers no) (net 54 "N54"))
  (pad "2" thru_hole oval (at 0 2.54) (size 1.7 1.7) (drill 1) (layers "*.Cu" "*.Mask") (remove_unused_layers no) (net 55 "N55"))
  (pad "3" thru_hole oval (at 0 5.08) (size 1.7 1.7) (drill 1) (layers "*.Cu" "*.Mask") (remove_unused_layers no) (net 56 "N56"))
  (pad "4" thru_hole oval (at 0 7.62) (size 1.7 1.7) (drill 1) (layers "*.Cu" "*.Mask") (remove_unused_layers no) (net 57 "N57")))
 (gr_rect (start 120.33 48.75) (end 141.33 99.75) (stroke (width 0.05) (type default)) (fill none) (layer "Edge.Cuts"))
 (segment (start 131.7225 54.991) (end 131.7225 53.285) (width 0.2) (layer "F.Cu") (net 53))
 (segment (start 131.7225 53.285) (end 129.8725 51.435) (width 0.2) (layer "F.Cu") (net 53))
 (segment (start 134.471 53.721) (end 135.89 55.14) (width 0.2) (layer "F.Cu") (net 7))
 (segment (start 131.7475 51.435) (end 133.096 51.435) (width 0.2) (layer "F.Cu") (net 7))
 (segment (start 133.096 51.435) (end 133.096 53.721) (width 0.2) (layer "F.Cu") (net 7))
 (segment (start 135.89 55.14) (end 139.7 55.14) (width 0.2) (layer "F.Cu") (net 7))
 (segment (start 133.096 53.721) (end 134.471 53.721) (width 0.2) (layer "F.Cu") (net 7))
 (segment (start 121.92 55.14) (end 125.73 55.14) (width 0.2) (layer "F.Cu") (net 35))
 (segment (start 125.73 67.84) (end 121.92 67.84) (width 0.2) (layer "F.Cu") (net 40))
 (segment (start 125.73 83.08) (end 121.92 83.08) (width 0.2) (layer "F.Cu") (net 46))
 (segment (start 125.73 57.68) (end 121.92 57.68) (width 0.2) (layer "F.Cu") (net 36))
 (segment (start 125.73 78) (end 121.92 78) (width 0.2) (layer "F.Cu") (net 44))
 (segment (start 121.92 90.7) (end 125.73 90.7) (width 0.2) (layer "F.Cu") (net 49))
 (segment (start 121.92 80.54) (end 125.73 80.54) (width 0.2) (layer "F.Cu") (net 45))
 (segment (start 121.92 95.78) (end 125.73 95.78) (width 0.2) (layer "F.Cu") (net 51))
 (segment (start 125.73 52.6) (end 121.92 52.6) (width 0.2) (layer "F.Cu") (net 34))
 (segment (start 121.92 85.62) (end 125.73 85.62) (width 0.2) (layer "F.Cu") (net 47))
 (segment (start 125.73 62.76) (end 121.92 62.76) (width 0.2) (layer "F.Cu") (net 38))
 (segment (start 121.92 75.46) (end 125.73 75.46) (width 0.2) (layer "F.Cu") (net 43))
 (segment (start 121.92 70.38) (end 125.73 70.38) (width 0.2) (layer "F.Cu") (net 41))
 (segment (start 125.73 98.32) (end 121.92 98.32) (width 0.2) (layer "F.Cu") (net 52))
 (segment (start 125.73 88.16) (end 121.92 88.16) (width 0.2) (layer "F.Cu") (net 48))
 (segment (start 125.73 93.24) (end 121.92 93.24) (width 0.2) (layer "F.Cu") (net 50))
 (segment (start 125.73 72.92) (end 121.92 72.92) (width 0.2) (layer "F.Cu") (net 42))
 (segment (start 121.92 60.22) (end 125.73 60.22) (width 0.2) (layer "F.Cu") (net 37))
 (segment (start 121.92 65.3) (end 125.73 65.3) (width 0.2) (layer "F.Cu") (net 39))
 (segment (start 121.92 50.06) (end 125.73 50.06) (width 0.2) (layer "F.Cu") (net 33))
 (segment (start 139.7 52.6) (end 135.89 52.6) (width 0.2) (layer "F.Cu") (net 6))
 (segment (start 139.7 78) (end 135.89 78) (width 0.2) (layer "F.Cu") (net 16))
 (segment (start 135.89 65.3) (end 139.7 65.3) (width 0.2) (layer "F.Cu") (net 11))
 (segment (start 139.7 57.68) (end 135.89 57.68) (width 0.2) (layer "F.Cu") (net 8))
 (segment (start 139.7 90.7) (end 135.89 90.7) (width 0.2) (layer "F.Cu") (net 21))
 (segment (start 135.89 98.32) (end 139.7 98.32) (width 0.2) (layer "F.Cu") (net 24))
 (segment (start 134.366 81.534) (end 134.896 81.534) (width 0.2) (layer "F.Cu") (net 17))
 (segment (start 134.896 81.534) (end 135.89 80.54) (width 0.2) (layer "F.Cu") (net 17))
 (segment (start 132.888 92.375) (end 132.969 92.456) (width 0.2) (layer "F.Cu") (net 17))
 (segment (start 139.7 80.54) (end 135.89 80.54) (width 0.2) (layer "F.Cu") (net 17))
 (segment (start 132.81 92.375) (end 132.81 85.63) (width 0.2) (layer "F.Cu") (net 17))
 (segment (start 132.81 92.375) (end 132.888 92.375) (width 0.2) (layer "F.Cu") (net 17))
 (segment (start 132.81 85.63) (end 134.366 84.074) (width 0.2) (layer "F.Cu") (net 17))
 (segment (start 134.366 84.074) (end 134.366 81.534) (width 0.2) (layer "F.Cu") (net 17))
 (segment (start 132.81 92.375) (end 132.81 98.125) (width 0.2) (layer "F.Cu") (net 17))
 (segment (start 139.7 72.92) (end 135.89 72.92) (width 0.2) (layer "F.Cu") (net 14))
 (segment (start 128.81 92.375) (end 128.81 87.979) (width 0.2) (layer "F.Cu") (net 15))
 (segment (start 128.81 92.375) (end 128.81 98.125) (width 0.2) (layer "F.Cu") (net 15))
 (segment (start 135.89 75.46) (end 139.7 75.46) (width 0.2) (layer "F.Cu") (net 15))
 (segment (start 131.064 85.725) (end 131.064 77.47) (width 0.2) (layer "F.Cu") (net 15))
 (segment (start 131.064 77.47) (end 133.88 77.47) (width 0.2) (layer "F.Cu") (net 15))
 (segment (start 133.88 77.47) (end 135.89 75.46) (width 0.2) (layer "F.Cu") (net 15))
 (segment (start 128.81 87.979) (end 131.064 85.725) (width 0.2) (layer "F.Cu") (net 15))
 (segment (start 135.89 93.24) (end 139.7 93.24) (width 0.2) (layer "F.Cu") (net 22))
 (segment (start 139.7 62.76) (end 135.89 62.76) (width 0.2) (layer "F.Cu") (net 10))
 (segment (start 139.7 67.84) (end 135.89 67.84) (width 0.2) (layer "F.Cu") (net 12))
 (segment (start 139.7 95.78) (end 135.89 95.78) (width 0.2) (layer "F.Cu") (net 23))
 (segment (start 135.89 60.22) (end 139.7 60.22) (width 0.2) (layer "F.Cu") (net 9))
 (segment (start 133.223 58.293) (end 133.477 58.547) (width 0.2) (layer "F.Cu") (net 9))
 (segment (start 129.8975 54.991) (end 129.8975 55.9835) (width 0.2) (layer "F.Cu") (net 9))
 (segment (start 133.223 56.769) (end 133.223 58.293) (width 0.2) (layer "F.Cu") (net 9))
 (segment (start 134.217 58.547) (end 135.89 60.22) (width 0.2) (layer "F.Cu") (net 9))
 (segment (start 129.8975 55.9835) (end 130.683 56.769) (width 0.2) (layer "F.Cu") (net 9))
 (segment (start 133.477 58.547) (end 134.217 58.547) (width 0.2) (layer "F.Cu") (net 9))
 (segment (start 130.683 56.769) (end 133.223 56.769) (width 0.2) (layer "F.Cu") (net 9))
 (segment (start 135.89 83.08) (end 139.7 83.08) (width 0.2) (layer "F.Cu") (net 18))
 (segment (start 135.89 88.16) (end 139.7 88.16) (width 0.2) (layer "F.Cu") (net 20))
 (segment (start 139.7 85.62) (end 135.89 85.62) (width 0.2) (layer "F.Cu") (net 19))
 (segment (start 135.89 50.06) (end 139.7 50.06) (width 0.2) (layer "F.Cu") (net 5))
 (segment (start 135.89 70.38) (end 139.7 70.38) (width 0.2) (layer "F.Cu") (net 13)))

